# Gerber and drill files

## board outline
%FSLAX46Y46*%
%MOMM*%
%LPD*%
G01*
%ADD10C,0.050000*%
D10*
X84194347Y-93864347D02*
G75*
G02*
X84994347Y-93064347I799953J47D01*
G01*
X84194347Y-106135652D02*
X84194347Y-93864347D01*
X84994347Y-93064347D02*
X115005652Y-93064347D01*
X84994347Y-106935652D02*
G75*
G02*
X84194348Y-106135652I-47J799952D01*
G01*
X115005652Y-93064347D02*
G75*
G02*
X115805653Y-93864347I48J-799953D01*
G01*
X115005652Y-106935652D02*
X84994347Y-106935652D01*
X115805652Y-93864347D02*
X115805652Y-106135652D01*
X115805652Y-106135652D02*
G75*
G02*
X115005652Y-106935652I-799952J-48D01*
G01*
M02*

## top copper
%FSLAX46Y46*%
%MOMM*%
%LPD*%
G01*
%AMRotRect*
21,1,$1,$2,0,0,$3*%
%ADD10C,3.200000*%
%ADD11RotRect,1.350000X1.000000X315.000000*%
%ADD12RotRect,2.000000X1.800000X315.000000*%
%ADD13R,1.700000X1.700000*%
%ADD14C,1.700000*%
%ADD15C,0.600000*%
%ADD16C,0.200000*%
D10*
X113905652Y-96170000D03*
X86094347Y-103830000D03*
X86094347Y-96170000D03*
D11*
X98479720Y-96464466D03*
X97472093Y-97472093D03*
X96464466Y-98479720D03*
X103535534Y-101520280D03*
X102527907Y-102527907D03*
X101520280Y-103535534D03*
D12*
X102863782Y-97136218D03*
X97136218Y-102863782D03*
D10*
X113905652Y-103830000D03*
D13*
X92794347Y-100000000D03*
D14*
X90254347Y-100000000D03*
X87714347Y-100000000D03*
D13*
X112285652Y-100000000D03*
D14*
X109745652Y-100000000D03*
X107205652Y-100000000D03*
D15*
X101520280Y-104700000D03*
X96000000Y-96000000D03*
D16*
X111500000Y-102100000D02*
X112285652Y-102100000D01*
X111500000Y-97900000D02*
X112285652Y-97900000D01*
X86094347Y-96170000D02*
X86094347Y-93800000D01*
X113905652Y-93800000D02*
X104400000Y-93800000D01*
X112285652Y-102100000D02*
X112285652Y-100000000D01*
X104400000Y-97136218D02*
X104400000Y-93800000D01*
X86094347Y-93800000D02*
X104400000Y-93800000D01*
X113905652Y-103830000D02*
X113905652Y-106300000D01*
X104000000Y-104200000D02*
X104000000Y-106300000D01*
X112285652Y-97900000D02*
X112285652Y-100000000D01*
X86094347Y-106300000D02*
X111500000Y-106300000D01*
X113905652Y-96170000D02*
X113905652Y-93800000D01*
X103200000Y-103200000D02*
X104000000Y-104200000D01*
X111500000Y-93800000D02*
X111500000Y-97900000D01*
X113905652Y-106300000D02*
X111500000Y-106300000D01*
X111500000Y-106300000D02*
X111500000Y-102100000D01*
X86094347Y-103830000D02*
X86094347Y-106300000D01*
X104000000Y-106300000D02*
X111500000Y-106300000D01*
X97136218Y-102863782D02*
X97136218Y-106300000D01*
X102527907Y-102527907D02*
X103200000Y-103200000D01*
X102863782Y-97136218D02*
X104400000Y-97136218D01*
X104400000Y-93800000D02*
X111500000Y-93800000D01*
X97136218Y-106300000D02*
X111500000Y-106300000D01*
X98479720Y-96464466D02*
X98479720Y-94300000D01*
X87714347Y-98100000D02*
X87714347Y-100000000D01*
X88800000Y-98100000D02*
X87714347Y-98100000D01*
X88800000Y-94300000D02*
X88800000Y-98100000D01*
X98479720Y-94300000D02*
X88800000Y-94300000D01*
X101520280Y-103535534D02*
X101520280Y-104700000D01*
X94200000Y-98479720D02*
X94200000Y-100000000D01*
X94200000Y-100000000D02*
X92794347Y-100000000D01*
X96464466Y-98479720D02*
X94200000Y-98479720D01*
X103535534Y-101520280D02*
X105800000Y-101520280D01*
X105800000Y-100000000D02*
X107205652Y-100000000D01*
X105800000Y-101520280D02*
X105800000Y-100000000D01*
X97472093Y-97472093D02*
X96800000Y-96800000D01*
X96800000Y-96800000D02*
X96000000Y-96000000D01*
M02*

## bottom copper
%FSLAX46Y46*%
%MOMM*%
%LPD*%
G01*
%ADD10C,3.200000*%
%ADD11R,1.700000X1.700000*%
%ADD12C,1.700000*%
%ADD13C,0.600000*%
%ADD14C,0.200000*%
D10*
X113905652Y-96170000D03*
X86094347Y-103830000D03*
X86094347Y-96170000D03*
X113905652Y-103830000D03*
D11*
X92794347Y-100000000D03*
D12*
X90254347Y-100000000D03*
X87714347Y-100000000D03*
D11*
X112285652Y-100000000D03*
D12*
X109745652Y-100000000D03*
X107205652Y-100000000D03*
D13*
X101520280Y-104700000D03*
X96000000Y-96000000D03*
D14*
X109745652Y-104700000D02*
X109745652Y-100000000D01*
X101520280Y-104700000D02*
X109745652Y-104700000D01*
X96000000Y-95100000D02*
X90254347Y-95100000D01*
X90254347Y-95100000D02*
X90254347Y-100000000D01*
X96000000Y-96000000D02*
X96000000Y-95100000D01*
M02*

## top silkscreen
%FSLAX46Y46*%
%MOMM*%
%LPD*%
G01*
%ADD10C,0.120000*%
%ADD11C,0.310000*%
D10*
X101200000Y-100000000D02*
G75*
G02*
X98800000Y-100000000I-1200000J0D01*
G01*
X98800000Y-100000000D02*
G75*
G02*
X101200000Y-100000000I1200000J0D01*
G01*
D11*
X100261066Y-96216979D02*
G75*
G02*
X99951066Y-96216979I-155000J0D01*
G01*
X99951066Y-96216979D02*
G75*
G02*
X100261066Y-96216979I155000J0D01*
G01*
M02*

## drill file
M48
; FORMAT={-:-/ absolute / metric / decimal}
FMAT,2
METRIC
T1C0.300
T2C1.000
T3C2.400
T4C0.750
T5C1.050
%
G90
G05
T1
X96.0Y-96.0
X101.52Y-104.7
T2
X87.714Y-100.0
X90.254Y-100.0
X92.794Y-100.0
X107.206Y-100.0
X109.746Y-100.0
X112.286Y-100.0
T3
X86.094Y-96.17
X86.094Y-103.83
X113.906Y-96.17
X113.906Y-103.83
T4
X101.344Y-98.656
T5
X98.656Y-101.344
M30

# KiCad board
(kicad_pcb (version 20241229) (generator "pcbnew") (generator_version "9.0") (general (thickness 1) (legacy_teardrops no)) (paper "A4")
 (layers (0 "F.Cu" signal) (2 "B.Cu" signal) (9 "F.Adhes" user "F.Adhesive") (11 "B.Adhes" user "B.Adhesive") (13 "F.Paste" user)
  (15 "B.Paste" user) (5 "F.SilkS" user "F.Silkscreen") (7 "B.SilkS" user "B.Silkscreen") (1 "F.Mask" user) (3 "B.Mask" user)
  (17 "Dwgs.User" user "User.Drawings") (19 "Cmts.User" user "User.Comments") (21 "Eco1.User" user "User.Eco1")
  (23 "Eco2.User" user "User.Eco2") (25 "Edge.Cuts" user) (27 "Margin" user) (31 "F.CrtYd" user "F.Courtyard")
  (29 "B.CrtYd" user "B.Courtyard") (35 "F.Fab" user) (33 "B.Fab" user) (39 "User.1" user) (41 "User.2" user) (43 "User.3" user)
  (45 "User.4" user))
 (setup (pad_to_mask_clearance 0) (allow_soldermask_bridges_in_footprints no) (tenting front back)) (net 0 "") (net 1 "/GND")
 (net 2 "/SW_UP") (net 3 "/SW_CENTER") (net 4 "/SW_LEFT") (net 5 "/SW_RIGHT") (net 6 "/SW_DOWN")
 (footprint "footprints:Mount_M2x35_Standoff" (layer "F.Cu") (at 113.905652 96.17)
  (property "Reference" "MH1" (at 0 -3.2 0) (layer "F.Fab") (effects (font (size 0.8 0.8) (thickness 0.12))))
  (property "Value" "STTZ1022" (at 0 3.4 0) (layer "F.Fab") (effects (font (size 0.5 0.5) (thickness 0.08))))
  (pad "1" thru_hole circle (at 0 0) (size 3.2 3.2) (drill 2.4) (layers "*.Cu" "*.Mask") (remove_unused_layers no) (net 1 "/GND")))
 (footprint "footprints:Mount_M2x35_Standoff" (layer "F.Cu") (at 86.094347 103.83)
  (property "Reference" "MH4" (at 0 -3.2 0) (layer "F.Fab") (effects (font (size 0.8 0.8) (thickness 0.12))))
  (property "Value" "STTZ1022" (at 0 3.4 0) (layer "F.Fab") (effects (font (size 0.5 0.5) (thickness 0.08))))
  (pad "1" thru_hole circle (at 0 0) (size 3.2 3.2) (drill 2.4) (layers "*.Cu" "*.Mask") (remove_unused_layers no) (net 1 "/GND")))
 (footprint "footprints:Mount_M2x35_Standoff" (layer "F.Cu") (at 86.094347 96.17)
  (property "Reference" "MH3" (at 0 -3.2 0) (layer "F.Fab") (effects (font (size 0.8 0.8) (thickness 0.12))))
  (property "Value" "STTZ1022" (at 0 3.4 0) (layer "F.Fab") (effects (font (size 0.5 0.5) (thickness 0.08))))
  (pad "1" thru_hole circle (at 0 0) (size 3.2 3.2) (drill 2.4) (layers "*.Cu" "*.Mask") (remove_unused_layers no) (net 1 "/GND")))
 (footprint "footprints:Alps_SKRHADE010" (layer "F.Cu") (at 100 100 -45)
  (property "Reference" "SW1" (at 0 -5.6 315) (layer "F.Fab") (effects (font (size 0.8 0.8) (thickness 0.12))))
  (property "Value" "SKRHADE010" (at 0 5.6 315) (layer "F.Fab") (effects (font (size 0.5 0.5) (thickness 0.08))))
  (fp_circle (center 0 0) (end 1.2 0) (stroke (width 0.12) (type solid)) (fill no) (layer "F.SilkS"))
  (fp_circle (center -2.6 -2.75) (end -2.35 -2.75) (stroke (width 0.12) (type solid)) (fill yes) (layer "F.SilkS"))
  (pad "" np_thru_hole circle (at 0 -1.9 315) (size 0.75 0.75) (drill 0.75) (layers "*.Cu" "*.Mask"))
  (pad "" np_thru_hole circle (at 0 1.9 315) (size 1.05 1.05) (drill 1.05) (layers "*.Cu" "*.Mask"))
  (pad "1" smd rect (at -3.575 -1.425 315) (size 1.35 1) (layers "F.Cu" "F.Mask" "F.Paste") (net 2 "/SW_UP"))
  (pad "2" smd rect (at -3.575 0 315) (size 1.35 1) (layers "F.Cu" "F.Mask" "F.Paste") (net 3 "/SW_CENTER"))
  (pad "3" smd rect (at -3.575 1.425 315) (size 1.35 1) (layers "F.Cu" "F.Mask" "F.Paste") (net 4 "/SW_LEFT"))
  (pad "4" smd rect (at 3.575 -1.425 315) (size 1.35 1) (layers "F.Cu" "F.Mask" "F.Paste") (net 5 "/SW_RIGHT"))
  (pad "5" smd rect (at 3.575 0 315) (size 1.35 1) (layers "F.Cu" "F.Mask" "F.Paste") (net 1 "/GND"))
  (pad "6" smd rect (at 3.575 1.425 315) (size 1.35 1) (layers "F.Cu" "F.Mask" "F.Paste") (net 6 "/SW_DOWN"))
  (pad "7" smd rect (at 0 -4.049999 315) (size 2 1.8) (layers "F.Cu" "F.Mask" "F.Paste") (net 1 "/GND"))
  (pad "8" smd rect (at 0 4.049999 315) (size 2 1.8) (layers "F.Cu" "F.Mask" "F.Paste") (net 1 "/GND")))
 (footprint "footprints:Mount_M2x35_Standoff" (layer "F.Cu") (at 113.905652 103.83)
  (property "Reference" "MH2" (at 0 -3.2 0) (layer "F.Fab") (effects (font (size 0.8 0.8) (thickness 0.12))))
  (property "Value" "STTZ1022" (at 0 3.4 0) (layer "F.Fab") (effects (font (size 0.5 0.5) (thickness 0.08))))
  (pad "1" thru_hole circle (at 0 0) (size 3.2 3.2) (drill 2.4) (layers "*.Cu" "*.Mask") (remove_unused_layers no) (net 1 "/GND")))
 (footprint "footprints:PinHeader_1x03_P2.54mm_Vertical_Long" (layer "B.Cu") (at 90.254347 100 180)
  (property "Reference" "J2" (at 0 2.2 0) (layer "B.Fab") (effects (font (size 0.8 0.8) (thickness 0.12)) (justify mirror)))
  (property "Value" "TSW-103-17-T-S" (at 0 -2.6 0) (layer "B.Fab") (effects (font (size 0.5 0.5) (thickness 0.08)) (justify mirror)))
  (pad "1" thru_hole rect (at -2.54 0 180) (size 1.7 1.7) (drill 1) (layers "*.Cu" "*.Mask") (remove_unused_layers no) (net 4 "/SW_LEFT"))
  (pad "2" thru_hole circle (at 0 0 180) (size 1.7 1.7) (drill 1) (layers "*.Cu" "*.Mask") (remove_unused_layers no) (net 3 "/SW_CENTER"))
  (pad "3" thru_hole circle (at 2.54 0 180) (size 1.7 1.7) (drill 1) (layers "*.Cu" "*.Mask") (remove_unused_layers no) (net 2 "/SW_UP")))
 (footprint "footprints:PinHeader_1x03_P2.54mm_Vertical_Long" (layer "B.Cu") (at 109.745652 100 180)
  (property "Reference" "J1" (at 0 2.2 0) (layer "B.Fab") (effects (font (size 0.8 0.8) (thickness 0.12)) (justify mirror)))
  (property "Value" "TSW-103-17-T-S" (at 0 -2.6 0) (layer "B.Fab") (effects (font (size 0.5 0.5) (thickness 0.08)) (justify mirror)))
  (pad "1" thru_hole rect (at -2.54 0 180) (size 1.7 1.7) (drill 1) (layers "*.Cu" "*.Mask") (remove_unused_layers no) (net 1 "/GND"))
  (pad "2" thru_hole circle (at 0 0 180) (size 1.7 1.7) (drill 1) (layers "*.Cu" "*.Mask") (remove_unused_layers no) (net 6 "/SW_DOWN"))
  (pad "3" thru_hole circle (at 2.54 0 180) (size 1.7 1.7) (drill 1) (layers "*.Cu" "*.Mask") (remove_unused_layers no) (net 5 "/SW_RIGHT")))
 (gr_arc (start 84.194347 93.864347) (mid 84.428662 93.298662) (end 84.994347 93.064347) (stroke (width 0.05) (type default))
  (layer "Edge.Cuts"))
 (gr_line (start 84.194347 106.135652) (end 84.194347 93.864347) (stroke (width 0.05) (type default)) (layer "Edge.Cuts"))
 (gr_line (start 84.994347 93.064347) (end 115.005652 93.064347) (stroke (width 0.05) (type default)) (layer "Edge.Cuts"))
 (gr_arc (start 84.994347 106.935652) (mid 84.428662 106.701337) (end 84.194347 106.135652) (stroke (width 0.05) (type default))
  (layer "Edge.Cuts"))
 (gr_arc (start 115.005652 93.064347) (mid 115.571337 93.298662) (end 115.805652 93.864347) (stroke (width 0.05) (type default))
  (layer "Edge.Cuts"))
 (gr_line (start 115.005652 106.935652) (end 84.994347 106.935652) (stroke (width 0.05) (type default)) (layer "Edge.Cuts"))
 (gr_line (start 115.805652 93.864347) (end 115.805652 106.135652) (stroke (width 0.05) (type default)) (layer "Edge.Cuts"))
 (gr_arc (start 115.805652 106.135652) (mid 115.571337 106.701337) (end 115.005652 106.935652) (stroke (width 0.05) (type default))
  (layer "Edge.Cuts"))
 (segment (start 111.5 102.1) (end 112.285652 102.1) (width 0.2) (layer "F.Cu") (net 1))
 (segment (start 111.5 97.9) (end 112.285652 97.9) (width 0.2) (layer "F.Cu") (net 1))
 (segment (start 86.094347 96.17) (end 86.094347 93.8) (width 0.2) (layer "F.Cu") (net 1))
 (segment (start 113.905652 93.8) (end 104.4 93.8) (width 0.2) (layer "F.Cu") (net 1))
 (segment (start 112.285652 102.1) (end 112.285652 100) (width 0.2) (layer "F.Cu") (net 1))
 (segment (start 104.4 97.136218) (end 104.4 93.8) (width 0.2) (layer "F.Cu") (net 1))
 (segment (start 86.094347 93.8) (end 104.4 93.8) (width 0.2) (layer "F.Cu") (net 1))
 (segment (start 113.905652 103.83) (end 113.905652 106.3) (width 0.2) (layer "F.Cu") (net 1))
 (segment (start 104 104.2) (end 104 106.3) (width 0.2) (layer "F.Cu") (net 1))
 (segment (start 112.285652 97.9) (end 112.285652 100) (width 0.2) (layer "F.Cu") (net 1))
 (segment (start 86.094347 106.3) (end 111.5 106.3) (width 0.2) (layer "F.Cu") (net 1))
 (segment (start 113.905652 96.17) (end 113.905652 93.8) (width 0.2) (layer "F.Cu") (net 1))
 (segment (start 103.2 103.2) (end 104 104.2) (width 0.2) (layer "F.Cu") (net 1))
 (segment (start 111.5 93.8) (end 111.5 97.9) (width 0.2) (layer "F.Cu") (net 1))
 (segment (start 113.905652 106.3) (end 111.5 106.3) (width 0.2) (layer "F.Cu") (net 1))
 (segment (start 111.5 106.3) (end 111.5 102.1) (width 0.2) (layer "F.Cu") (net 1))
 (segment (start 86.094347 103.83) (end 86.094347 106.3) (width 0.2) (layer "F.Cu") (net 1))
 (segment (start 104 106.3) (end 111.5 106.3) (width 0.2) (layer "F.Cu") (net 1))
 (segment (start 97.136218 102.863782) (end 97.136218 106.3) (width 0.2) (layer "F.Cu") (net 1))
 (segment (start 102.527907 102.527907) (end 103.2 103.2) (width 0.2) (layer "F.Cu") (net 1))
 (segment (start 102.863782 97.136218) (end 104.4 97.136218) (width 0.2) (layer "F.Cu") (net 1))
 (segment (start 104.4 93.8) (end 111.5 93.8) (width 0.2) (layer "F.Cu") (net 1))
 (segment (start 97.136218 106.3) (end 111.5 106.3) (width 0.2) (layer "F.Cu") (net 1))
 (segment (start 98.47972 96.464466) (end 98.47972 94.3) (width 0.2) (layer "F.Cu") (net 2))
 (segment (start 87.714347 98.1) (end 87.714347 100) (width 0.2) (layer "F.Cu") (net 2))
 (segment (start 88.8 98.1) (end 87.714347 98.1) (width 0.2) (layer "F.Cu") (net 2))
 (segment (start 88.8 94.3) (end 88.8 98.1) (width 0.2) (layer "F.Cu") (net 2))
 (segment (start 98.47972 94.3) (end 88.8 94.3) (width 0.2) (layer "F.Cu") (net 2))
 (segment (start 101.52028 103.535534) (end 101.52028 104.7) (width 0.2) (layer "F.Cu") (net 6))
 (via (at 101.52028 104.7) (size 0.6) (drill 0.3) (layers "F.Cu" "B.Cu") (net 6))
 (segment (start 109.745652 104.7) (end 109.745652 100) (width 0.2) (layer "B.Cu") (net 6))
 (segment (start 101.52028 104.7) (end 109.745652 104.7) (width 0.2) (layer "B.Cu") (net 6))
 (segment (start 94.2 98.47972) (end 94.2 100) (width 0.2) (layer "F.Cu") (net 4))
 (segment (start 94.2 100) (end 92.794347 100) (width 0.2) (layer "F.Cu") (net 4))
 (segment (start 96.464466 98.47972) (end 94.2 98.47972) (width 0.2) (layer "F.Cu") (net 4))
 (segment (start 103.535534 101.52028) (end 105.8 101.52028) (width 0.2) (layer "F.Cu") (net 5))
 (segment (start 105.8 100) (end 107.205652 100) (width 0.2) (layer "F.Cu") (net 5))
 (segment (start 105.8 101.52028) (end 105.8 100) (width 0.2) (layer "F.Cu") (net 5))
 (segment (start 97.472093 97.472093) (end 96.8 96.8) (width 0.2) (layer "F.Cu") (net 3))
 (segment (start 96.8 96.8) (end 96 96) (width 0.2) (layer "F.Cu") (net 3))
 (via (at 96 96) (size 0.6) (drill 0.3) (layers "F.Cu" "B.Cu") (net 3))
 (segment (start 96 95.1) (end 90.254347 95.1) (width 0.2) (layer "B.Cu") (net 3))
 (segment (start 90.254347 95.1) (end 90.254347 100) (width 0.2) (layer "B.Cu") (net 3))
 (segment (start 96 96) (end 96 95.1) (width 0.2) (layer "B.Cu") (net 3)))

